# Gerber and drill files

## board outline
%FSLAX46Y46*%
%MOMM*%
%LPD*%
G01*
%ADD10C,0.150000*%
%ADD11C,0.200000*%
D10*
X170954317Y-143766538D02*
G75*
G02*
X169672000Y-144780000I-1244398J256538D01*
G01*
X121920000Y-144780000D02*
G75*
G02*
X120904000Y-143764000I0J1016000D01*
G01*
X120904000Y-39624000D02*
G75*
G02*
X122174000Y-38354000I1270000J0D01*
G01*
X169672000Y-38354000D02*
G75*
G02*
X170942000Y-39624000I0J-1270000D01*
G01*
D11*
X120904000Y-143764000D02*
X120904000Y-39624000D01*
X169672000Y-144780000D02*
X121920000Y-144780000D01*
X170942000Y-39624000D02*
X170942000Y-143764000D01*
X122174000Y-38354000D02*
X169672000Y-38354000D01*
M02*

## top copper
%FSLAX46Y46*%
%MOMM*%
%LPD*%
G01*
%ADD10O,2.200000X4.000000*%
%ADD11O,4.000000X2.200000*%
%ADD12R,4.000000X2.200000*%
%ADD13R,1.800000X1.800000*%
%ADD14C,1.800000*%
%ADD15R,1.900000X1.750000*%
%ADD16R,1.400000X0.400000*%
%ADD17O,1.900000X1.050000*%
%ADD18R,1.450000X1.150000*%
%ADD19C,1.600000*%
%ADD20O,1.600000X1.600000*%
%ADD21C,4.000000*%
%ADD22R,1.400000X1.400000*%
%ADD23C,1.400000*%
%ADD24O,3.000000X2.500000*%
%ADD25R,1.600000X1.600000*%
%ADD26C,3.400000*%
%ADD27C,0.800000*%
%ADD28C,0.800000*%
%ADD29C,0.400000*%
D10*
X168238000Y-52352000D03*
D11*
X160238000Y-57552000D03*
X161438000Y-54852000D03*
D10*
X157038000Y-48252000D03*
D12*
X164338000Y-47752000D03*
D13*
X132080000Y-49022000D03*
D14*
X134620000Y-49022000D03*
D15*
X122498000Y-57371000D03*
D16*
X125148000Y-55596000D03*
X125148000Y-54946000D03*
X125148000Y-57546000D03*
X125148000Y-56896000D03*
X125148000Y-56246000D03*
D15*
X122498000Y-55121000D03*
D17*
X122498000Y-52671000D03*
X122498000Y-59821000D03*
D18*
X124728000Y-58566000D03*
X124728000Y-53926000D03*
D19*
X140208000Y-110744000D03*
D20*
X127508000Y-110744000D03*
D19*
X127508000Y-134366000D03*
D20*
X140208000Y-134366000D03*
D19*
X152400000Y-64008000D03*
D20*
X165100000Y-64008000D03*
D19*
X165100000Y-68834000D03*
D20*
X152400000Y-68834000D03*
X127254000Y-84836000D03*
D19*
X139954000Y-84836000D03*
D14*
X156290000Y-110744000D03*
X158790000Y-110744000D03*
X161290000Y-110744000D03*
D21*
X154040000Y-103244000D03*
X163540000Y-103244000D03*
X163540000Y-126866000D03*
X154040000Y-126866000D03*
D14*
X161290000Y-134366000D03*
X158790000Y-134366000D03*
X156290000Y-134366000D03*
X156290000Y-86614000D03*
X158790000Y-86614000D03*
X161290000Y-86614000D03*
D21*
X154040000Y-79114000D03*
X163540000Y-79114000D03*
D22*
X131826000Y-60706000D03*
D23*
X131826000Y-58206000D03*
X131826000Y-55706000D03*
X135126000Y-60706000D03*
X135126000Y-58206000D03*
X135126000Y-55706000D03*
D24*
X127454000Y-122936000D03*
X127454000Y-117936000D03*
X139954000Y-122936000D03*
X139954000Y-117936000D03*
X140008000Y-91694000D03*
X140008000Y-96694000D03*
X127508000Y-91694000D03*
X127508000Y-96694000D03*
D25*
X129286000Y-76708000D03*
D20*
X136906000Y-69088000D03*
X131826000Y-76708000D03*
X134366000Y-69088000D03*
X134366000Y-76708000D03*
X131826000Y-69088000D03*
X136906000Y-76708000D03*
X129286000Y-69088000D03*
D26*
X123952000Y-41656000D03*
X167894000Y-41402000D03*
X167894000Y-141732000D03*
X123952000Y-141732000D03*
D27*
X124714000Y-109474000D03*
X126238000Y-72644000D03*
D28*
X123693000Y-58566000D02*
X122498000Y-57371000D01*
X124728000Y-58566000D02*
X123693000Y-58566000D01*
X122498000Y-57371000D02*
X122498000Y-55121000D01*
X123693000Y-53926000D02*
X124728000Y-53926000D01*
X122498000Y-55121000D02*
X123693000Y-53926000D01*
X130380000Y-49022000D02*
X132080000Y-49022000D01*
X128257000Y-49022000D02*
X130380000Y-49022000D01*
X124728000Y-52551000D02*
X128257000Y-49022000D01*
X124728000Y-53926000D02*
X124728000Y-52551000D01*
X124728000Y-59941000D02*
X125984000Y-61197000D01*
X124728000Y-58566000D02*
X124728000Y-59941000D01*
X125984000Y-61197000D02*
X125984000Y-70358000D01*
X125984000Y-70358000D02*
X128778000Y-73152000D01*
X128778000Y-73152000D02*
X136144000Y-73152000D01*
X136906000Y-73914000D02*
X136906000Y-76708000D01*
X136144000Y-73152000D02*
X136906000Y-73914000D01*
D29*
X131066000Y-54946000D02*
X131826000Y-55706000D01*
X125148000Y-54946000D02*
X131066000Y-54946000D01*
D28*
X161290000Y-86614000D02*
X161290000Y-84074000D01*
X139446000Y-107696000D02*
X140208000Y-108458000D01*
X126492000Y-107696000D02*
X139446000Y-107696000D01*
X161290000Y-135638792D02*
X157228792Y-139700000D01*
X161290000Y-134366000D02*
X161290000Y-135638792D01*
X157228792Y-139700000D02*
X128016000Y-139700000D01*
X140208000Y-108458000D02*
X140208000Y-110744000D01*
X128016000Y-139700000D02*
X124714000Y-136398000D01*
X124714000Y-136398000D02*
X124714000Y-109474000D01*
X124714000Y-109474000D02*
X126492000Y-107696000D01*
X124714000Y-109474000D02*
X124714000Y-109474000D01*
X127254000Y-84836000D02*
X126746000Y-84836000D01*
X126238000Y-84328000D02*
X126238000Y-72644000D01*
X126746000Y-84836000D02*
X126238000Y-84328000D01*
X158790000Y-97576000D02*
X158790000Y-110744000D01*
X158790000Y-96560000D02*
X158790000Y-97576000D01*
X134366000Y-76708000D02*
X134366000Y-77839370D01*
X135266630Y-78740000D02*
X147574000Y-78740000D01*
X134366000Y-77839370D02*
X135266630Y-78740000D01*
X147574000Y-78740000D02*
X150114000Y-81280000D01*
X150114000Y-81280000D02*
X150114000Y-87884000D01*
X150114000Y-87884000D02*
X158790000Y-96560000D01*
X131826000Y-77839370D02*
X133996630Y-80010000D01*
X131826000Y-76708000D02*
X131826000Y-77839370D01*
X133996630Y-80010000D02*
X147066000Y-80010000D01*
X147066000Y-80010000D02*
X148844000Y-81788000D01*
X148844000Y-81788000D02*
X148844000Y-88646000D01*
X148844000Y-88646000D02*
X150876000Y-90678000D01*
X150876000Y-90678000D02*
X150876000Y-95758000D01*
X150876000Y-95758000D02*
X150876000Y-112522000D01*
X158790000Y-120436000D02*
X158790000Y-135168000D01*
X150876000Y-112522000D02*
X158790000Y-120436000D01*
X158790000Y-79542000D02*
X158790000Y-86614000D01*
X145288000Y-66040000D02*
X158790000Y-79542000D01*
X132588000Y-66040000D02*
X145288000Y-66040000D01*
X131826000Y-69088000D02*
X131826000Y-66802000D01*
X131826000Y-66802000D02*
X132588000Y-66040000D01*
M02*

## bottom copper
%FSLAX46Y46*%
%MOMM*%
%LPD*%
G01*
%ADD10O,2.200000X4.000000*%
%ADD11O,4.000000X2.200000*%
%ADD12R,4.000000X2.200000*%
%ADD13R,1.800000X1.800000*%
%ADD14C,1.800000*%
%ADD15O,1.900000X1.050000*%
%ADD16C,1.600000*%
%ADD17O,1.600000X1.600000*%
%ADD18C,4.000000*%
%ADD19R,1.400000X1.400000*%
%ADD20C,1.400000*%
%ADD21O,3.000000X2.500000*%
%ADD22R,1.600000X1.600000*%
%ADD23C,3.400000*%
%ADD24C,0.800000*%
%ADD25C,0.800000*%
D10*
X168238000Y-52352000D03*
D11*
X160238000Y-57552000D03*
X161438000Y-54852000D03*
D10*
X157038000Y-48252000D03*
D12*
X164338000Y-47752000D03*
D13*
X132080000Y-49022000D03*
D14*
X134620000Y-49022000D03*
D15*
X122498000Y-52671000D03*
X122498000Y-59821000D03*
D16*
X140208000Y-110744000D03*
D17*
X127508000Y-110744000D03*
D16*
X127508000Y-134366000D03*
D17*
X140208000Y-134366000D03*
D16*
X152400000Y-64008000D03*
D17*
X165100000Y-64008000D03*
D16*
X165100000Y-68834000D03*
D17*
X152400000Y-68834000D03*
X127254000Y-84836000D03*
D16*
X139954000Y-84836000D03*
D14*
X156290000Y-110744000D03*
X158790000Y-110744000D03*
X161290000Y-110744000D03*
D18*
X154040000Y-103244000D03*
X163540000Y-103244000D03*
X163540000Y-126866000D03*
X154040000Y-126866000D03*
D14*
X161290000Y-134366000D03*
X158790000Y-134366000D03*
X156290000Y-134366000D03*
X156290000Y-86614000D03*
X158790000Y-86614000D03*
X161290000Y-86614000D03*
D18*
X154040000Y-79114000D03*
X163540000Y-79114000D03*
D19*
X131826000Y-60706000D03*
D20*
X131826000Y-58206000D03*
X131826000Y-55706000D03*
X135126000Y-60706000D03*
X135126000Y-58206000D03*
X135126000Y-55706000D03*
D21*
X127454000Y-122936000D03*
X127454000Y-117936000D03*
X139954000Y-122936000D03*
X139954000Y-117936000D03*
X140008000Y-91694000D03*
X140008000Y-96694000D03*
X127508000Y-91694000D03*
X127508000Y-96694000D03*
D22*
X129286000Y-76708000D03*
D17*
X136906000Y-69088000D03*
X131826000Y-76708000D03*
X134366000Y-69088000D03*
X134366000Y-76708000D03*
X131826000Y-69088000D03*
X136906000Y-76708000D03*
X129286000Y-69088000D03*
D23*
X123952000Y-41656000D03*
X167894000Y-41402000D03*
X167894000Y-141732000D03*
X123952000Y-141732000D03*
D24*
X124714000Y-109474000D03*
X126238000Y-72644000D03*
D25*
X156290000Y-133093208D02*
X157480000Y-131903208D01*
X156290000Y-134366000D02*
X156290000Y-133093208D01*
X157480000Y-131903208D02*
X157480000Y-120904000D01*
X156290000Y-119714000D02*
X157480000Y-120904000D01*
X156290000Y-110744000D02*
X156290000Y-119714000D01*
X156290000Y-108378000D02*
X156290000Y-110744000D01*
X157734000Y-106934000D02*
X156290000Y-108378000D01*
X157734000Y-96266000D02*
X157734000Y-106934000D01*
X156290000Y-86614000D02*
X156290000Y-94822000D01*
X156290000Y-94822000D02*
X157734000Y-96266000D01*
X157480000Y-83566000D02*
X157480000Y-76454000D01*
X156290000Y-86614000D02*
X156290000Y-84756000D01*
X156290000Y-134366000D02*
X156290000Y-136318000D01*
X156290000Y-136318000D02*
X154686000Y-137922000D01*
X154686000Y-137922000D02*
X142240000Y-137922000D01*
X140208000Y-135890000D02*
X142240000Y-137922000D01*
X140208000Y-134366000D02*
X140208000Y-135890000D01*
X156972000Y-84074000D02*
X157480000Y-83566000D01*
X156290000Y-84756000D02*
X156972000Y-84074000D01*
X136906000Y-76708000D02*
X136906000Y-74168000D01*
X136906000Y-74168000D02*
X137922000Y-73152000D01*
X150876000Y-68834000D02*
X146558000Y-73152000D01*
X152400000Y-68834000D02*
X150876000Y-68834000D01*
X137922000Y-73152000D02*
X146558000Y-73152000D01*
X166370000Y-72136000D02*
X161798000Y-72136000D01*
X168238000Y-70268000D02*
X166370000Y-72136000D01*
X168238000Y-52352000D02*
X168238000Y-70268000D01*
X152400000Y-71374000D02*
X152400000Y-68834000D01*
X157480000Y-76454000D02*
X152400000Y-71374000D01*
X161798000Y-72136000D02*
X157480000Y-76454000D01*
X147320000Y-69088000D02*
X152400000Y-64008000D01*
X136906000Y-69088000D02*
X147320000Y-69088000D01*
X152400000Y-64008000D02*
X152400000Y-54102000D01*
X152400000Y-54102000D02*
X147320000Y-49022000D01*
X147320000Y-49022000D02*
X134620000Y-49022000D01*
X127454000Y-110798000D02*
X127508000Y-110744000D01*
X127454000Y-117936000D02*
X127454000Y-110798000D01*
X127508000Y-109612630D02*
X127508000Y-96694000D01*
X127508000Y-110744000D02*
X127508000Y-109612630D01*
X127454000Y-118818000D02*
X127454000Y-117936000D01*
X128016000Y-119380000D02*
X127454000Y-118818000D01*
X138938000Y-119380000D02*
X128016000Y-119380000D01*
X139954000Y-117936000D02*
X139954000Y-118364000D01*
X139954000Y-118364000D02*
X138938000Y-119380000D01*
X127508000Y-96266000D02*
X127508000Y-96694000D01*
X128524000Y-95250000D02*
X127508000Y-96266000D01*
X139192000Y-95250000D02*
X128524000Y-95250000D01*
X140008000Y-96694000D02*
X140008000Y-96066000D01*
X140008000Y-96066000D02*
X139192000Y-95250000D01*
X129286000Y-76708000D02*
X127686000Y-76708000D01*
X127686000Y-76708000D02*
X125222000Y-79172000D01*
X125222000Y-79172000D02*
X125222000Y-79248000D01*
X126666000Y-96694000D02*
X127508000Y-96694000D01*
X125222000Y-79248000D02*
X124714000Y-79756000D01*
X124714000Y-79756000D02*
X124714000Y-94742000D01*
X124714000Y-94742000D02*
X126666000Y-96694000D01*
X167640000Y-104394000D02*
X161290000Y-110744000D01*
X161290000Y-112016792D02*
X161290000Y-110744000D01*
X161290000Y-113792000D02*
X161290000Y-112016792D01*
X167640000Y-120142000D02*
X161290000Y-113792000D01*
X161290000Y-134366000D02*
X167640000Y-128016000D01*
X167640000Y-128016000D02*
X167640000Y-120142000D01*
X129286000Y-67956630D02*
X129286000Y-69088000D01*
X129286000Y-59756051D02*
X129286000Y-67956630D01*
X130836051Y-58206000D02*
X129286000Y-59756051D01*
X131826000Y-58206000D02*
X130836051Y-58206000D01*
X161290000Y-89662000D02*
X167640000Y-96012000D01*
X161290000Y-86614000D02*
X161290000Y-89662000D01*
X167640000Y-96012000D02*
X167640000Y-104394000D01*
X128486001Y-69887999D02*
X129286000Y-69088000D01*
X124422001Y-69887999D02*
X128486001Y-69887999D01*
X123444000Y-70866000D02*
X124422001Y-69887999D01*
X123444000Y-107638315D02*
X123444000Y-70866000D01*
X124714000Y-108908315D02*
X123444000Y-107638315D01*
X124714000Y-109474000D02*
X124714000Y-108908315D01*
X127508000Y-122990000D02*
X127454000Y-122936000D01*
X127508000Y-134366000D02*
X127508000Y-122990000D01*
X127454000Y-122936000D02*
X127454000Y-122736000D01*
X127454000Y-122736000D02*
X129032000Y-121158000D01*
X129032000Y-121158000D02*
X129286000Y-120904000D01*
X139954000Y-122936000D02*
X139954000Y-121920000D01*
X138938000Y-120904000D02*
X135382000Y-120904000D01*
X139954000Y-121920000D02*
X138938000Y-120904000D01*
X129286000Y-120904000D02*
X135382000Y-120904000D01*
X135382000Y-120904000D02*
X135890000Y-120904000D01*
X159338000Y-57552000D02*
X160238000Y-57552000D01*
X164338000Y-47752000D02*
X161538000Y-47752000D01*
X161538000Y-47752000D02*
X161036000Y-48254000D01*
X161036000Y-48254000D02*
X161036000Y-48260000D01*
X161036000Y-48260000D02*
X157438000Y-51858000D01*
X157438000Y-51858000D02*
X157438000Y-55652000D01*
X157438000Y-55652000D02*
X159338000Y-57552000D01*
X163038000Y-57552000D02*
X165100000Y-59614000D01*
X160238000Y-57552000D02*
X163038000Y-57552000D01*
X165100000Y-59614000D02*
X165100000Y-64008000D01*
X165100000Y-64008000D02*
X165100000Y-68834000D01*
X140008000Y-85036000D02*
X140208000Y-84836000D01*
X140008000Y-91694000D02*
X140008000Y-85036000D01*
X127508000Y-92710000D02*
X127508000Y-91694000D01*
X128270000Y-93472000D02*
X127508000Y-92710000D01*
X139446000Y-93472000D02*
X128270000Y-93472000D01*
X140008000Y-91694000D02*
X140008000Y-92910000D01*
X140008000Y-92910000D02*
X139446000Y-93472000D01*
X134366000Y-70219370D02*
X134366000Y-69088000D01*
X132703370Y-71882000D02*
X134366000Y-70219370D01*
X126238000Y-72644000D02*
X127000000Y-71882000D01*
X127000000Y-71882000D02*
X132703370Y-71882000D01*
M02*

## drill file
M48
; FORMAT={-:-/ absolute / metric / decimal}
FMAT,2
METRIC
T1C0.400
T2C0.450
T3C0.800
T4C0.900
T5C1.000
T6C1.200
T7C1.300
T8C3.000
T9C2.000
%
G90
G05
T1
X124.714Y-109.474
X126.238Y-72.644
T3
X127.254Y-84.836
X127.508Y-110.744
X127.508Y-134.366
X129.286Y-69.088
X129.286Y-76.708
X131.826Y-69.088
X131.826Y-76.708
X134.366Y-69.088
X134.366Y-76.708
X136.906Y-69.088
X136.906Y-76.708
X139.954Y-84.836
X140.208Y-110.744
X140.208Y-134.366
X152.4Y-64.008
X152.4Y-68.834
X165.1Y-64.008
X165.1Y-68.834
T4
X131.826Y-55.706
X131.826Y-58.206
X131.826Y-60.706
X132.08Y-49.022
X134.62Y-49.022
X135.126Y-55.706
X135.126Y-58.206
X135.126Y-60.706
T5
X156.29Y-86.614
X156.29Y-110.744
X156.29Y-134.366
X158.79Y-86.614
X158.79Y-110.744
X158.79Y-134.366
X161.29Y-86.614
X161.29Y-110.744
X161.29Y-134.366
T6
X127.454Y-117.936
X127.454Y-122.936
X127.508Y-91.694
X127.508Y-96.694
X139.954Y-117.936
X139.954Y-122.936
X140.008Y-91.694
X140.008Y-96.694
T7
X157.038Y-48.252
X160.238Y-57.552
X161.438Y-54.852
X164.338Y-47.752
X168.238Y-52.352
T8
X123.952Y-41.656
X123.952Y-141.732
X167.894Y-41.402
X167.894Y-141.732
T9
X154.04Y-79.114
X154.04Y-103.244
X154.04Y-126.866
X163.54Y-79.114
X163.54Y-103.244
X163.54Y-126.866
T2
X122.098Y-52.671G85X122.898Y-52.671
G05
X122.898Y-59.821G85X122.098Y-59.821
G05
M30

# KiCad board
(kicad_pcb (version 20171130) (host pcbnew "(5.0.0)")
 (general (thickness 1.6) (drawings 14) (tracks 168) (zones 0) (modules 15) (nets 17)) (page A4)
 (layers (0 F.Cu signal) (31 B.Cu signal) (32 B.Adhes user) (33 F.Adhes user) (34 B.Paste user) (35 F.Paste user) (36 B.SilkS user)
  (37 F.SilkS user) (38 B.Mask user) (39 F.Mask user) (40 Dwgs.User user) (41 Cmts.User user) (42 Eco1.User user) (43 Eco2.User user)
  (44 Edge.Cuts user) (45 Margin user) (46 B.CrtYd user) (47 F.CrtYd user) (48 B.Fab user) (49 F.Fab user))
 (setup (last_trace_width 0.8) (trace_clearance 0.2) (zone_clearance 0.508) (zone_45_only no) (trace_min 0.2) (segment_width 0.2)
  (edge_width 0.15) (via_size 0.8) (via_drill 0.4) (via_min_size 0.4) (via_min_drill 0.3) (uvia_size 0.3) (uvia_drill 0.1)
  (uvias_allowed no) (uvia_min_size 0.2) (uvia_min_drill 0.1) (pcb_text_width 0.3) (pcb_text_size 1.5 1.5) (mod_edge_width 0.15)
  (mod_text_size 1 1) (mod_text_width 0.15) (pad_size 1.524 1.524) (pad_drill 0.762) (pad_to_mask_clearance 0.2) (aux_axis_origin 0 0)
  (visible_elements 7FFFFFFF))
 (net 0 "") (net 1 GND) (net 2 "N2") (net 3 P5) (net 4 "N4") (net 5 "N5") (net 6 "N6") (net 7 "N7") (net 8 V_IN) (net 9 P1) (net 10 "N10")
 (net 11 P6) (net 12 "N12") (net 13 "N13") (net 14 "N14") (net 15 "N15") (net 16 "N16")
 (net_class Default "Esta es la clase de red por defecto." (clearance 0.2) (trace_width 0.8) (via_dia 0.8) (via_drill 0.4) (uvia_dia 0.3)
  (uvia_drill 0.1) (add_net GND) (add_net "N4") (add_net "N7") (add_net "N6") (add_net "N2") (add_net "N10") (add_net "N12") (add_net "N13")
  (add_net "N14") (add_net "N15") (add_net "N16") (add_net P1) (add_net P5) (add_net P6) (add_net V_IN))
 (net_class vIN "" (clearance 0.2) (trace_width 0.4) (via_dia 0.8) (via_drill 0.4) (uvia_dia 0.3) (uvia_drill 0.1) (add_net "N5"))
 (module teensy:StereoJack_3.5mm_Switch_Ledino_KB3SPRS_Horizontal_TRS (layer F.Cu) (at 164.338 47.752 180)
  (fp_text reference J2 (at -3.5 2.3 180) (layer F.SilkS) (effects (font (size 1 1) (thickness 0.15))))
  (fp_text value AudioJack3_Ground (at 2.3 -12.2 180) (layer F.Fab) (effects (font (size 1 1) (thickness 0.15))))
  (pad S thru_hole oval (at -3.9 -4.6 180) (size 2.2 4) (drill 1.3) (layers *.Cu *.Mask) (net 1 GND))
  (pad T thru_hole oval (at 4.1 -9.8 180) (size 4 2.2) (drill 1.3) (layers *.Cu *.Mask) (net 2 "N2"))
  (pad 5 thru_hole oval (at 2.9 -7.1 180) (size 4 2.2) (drill 1.3) (layers *.Cu *.Mask))
  (pad 4 thru_hole oval (at 7.3 -0.5 270) (size 4 2.2) (drill 1.3) (layers *.Cu *.Mask))
  (pad R thru_hole rect (at 0 0 180) (size 4 2.2) (drill 1.3) (layers *.Cu *.Mask) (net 2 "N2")))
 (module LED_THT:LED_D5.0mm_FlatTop (layer F.Cu) (at 132.08 49.022)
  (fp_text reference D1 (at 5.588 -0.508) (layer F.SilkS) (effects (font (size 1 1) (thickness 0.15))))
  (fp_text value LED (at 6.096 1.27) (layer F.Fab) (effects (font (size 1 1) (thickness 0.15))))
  (pad 1 thru_hole rect (at 0 0) (size 1.8 1.8) (drill 0.9) (layers *.Cu *.Mask) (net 1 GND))
  (pad 2 thru_hole circle (at 2.54 0) (size 1.8 1.8) (drill 0.9) (layers *.Cu *.Mask) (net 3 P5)))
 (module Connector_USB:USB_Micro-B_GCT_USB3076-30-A (layer F.Cu) (at 123.698 56.246 270)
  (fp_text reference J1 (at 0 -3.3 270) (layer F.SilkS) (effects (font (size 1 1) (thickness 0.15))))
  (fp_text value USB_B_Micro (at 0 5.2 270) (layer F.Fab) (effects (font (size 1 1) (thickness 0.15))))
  (pad 6 smd rect (at 1.125 1.2 270) (size 1.75 1.9) (layers F.Cu F.Paste F.Mask) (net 1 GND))
  (pad 2 smd rect (at -0.65 -1.45 270) (size 0.4 1.4) (layers F.Cu F.Paste F.Mask) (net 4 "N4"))
  (pad 1 smd rect (at -1.3 -1.45 270) (size 0.4 1.4) (layers F.Cu F.Paste F.Mask) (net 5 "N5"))
  (pad 5 smd rect (at 1.3 -1.45 270) (size 0.4 1.4) (layers F.Cu F.Paste F.Mask) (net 1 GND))
  (pad 4 smd rect (at 0.65 -1.45 270) (size 0.4 1.4) (layers F.Cu F.Paste F.Mask) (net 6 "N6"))
  (pad 3 smd rect (at 0 -1.45 270) (size 0.4 1.4) (layers F.Cu F.Paste F.Mask) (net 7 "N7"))
  (pad 6 smd rect (at -1.125 1.2 270) (size 1.75 1.9) (layers F.Cu F.Paste F.Mask) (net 1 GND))
  (pad 6 thru_hole oval (at -3.575 1.2 90) (size 1.05 1.9) (drill oval 0.45 1.25) (layers *.Cu *.Mask) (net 1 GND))
  (pad 6 thru_hole oval (at 3.575 1.2 270) (size 1.05 1.9) (drill oval 0.45 1.25) (layers *.Cu *.Mask) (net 1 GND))
  (pad 6 smd rect (at 2.32 -1.03 270) (size 1.15 1.45) (layers F.Cu F.Paste F.Mask) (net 1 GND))
  (pad 6 smd rect (at -2.32 -1.03 270) (size 1.15 1.45) (layers F.Cu F.Paste F.Mask) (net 1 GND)))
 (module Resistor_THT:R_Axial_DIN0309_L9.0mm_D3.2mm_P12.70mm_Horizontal (layer F.Cu) (at 140.208 110.744 180)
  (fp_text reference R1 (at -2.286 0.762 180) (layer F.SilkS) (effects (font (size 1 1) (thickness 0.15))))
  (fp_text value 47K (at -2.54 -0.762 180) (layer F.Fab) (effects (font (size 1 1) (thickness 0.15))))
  (pad 1 thru_hole circle (at 0 0 180) (size 1.6 1.6) (drill 0.8) (layers *.Cu *.Mask) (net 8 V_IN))
  (pad 2 thru_hole oval (at 12.7 0 180) (size 1.6 1.6) (drill 0.8) (layers *.Cu *.Mask) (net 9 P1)))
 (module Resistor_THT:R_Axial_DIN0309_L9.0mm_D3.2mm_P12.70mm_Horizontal (layer F.Cu) (at 127.508 134.366)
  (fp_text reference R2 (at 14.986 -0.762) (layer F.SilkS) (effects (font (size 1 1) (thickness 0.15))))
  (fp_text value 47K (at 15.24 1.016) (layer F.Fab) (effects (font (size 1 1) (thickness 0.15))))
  (pad 1 thru_hole circle (at 0 0) (size 1.6 1.6) (drill 0.8) (layers *.Cu *.Mask) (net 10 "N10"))
  (pad 2 thru_hole oval (at 12.7 0) (size 1.6 1.6) (drill 0.8) (layers *.Cu *.Mask) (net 1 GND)))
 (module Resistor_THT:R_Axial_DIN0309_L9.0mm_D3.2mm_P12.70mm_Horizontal (layer F.Cu) (at 152.4 64.008)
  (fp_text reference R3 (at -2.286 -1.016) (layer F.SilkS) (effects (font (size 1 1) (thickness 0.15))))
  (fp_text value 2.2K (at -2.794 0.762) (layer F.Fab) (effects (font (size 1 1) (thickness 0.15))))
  (pad 1 thru_hole circle (at 0 0) (size 1.6 1.6) (drill 0.8) (layers *.Cu *.Mask) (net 3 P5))
  (pad 2 thru_hole oval (at 12.7 0) (size 1.6 1.6) (drill 0.8) (layers *.Cu *.Mask) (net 2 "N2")))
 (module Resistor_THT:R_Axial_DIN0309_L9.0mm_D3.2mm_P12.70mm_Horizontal (layer F.Cu) (at 165.1 68.834 180)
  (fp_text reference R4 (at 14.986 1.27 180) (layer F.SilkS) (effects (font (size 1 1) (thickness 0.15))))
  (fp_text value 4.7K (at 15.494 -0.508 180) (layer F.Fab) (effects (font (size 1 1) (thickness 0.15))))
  (pad 1 thru_hole circle (at 0 0 180) (size 1.6 1.6) (drill 0.8) (layers *.Cu *.Mask) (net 2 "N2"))
  (pad 2 thru_hole oval (at 12.7 0 180) (size 1.6 1.6) (drill 0.8) (layers *.Cu *.Mask) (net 1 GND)))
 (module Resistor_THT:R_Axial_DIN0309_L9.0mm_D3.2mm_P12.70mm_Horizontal (layer F.Cu) (at 139.954 84.836 180)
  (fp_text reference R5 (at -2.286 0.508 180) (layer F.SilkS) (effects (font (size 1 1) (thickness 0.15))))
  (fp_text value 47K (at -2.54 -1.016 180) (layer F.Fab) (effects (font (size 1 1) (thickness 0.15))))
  (pad 2 thru_hole oval (at 12.7 0 180) (size 1.6 1.6) (drill 0.8) (layers *.Cu *.Mask) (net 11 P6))
  (pad 1 thru_hole circle (at 0 0 180) (size 1.6 1.6) (drill 0.8) (layers *.Cu *.Mask) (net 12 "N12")))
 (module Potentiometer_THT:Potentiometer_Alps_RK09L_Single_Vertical (layer F.Cu) (at 161.29 110.744 90)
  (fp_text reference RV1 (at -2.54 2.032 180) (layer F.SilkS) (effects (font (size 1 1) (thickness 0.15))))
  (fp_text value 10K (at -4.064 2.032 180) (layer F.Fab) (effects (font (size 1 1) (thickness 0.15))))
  (pad 3 thru_hole circle (at 0 -5 90) (size 1.8 1.8) (drill 1) (layers *.Cu *.Mask) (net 1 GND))
  (pad 2 thru_hole circle (at 0 -2.5 90) (size 1.8 1.8) (drill 1) (layers *.Cu *.Mask) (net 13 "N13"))
  (pad 1 thru_hole circle (at 0 0 90) (size 1.8 1.8) (drill 1) (layers *.Cu *.Mask) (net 8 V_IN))
  (pad "" np_thru_hole circle (at 7.5 -7.25 90) (size 4 4) (drill 2) (layers *.Cu *.Mask))
  (pad "" np_thru_hole circle (at 7.5 2.25 90) (size 4 4) (drill 2) (layers *.Cu *.Mask)))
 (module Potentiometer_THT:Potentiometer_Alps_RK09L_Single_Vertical (layer F.Cu) (at 161.29 134.366 90)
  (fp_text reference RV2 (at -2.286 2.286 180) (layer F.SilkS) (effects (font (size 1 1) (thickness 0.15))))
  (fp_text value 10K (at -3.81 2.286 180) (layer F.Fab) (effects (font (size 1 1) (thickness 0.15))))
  (pad "" np_thru_hole circle (at 7.5 2.25 90) (size 4 4) (drill 2) (layers *.Cu *.Mask))
  (pad "" np_thru_hole circle (at 7.5 -7.25 90) (size 4 4) (drill 2) (layers *.Cu *.Mask))
  (pad 1 thru_hole circle (at 0 0 90) (size 1.8 1.8) (drill 1) (layers *.Cu *.Mask) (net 8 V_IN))
  (pad 2 thru_hole circle (at 0 -2.5 90) (size 1.8 1.8) (drill 1) (layers *.Cu *.Mask) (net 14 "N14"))
  (pad 3 thru_hole circle (at 0 -5 90) (size 1.8 1.8) (drill 1) (layers *.Cu *.Mask) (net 1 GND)))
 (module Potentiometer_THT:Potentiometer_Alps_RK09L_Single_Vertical (layer F.Cu) (at 161.29 86.614 90)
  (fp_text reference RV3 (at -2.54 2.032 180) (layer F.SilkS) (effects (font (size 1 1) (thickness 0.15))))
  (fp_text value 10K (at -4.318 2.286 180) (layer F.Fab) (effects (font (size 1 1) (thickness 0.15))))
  (pad 3 thru_hole circle (at 0 -5 90) (size 1.8 1.8) (drill 1) (layers *.Cu *.Mask) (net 1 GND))
  (pad 2 thru_hole circle (at 0 -2.5 90) (size 1.8 1.8) (drill 1) (layers *.Cu *.Mask) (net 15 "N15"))
  (pad 1 thru_hole circle (at 0 0 90) (size 1.8 1.8) (drill 1) (layers *.Cu *.Mask) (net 8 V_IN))
  (pad "" np_thru_hole circle (at 7.5 -7.25 90) (size 4 4) (drill 2) (layers *.Cu *.Mask))
  (pad "" np_thru_hole circle (at 7.5 2.25 90) (size 4 4) (drill 2) (layers *.Cu *.Mask)))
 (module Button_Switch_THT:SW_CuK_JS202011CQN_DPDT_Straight (layer F.Cu) (at 131.826 60.706 90)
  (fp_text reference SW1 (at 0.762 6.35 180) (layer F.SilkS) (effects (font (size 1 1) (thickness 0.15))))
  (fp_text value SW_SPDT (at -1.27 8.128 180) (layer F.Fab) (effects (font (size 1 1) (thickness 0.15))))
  (pad 1 thru_hole rect (at 0 0 90) (size 1.4 1.4) (drill 0.9) (layers *.Cu *.Mask) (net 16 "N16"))
  (pad 2 thru_hole circle (at 2.5 0 90) (size 1.4 1.4) (drill 0.9) (layers *.Cu *.Mask) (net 8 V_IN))
  (pad 3 thru_hole circle (at 5 0 90) (size 1.4 1.4) (drill 0.9) (layers *.Cu *.Mask) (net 5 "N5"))
  (pad 4 thru_hole circle (at 0 3.3 90) (size 1.4 1.4) (drill 0.9) (layers *.Cu *.Mask))
  (pad 5 thru_hole circle (at 2.5 3.3 90) (size 1.4 1.4) (drill 0.9) (layers *.Cu *.Mask))
  (pad 6 thru_hole circle (at 5 3.3 90) (size 1.4 1.4) (drill 0.9) (layers *.Cu *.Mask)))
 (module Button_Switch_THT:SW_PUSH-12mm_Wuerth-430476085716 (layer F.Cu) (at 139.954 122.936 180)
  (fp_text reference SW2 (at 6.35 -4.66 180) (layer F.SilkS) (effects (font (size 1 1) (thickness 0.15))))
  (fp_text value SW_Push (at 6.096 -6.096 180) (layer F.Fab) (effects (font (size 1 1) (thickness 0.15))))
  (pad 1 thru_hole oval (at 12.5 0 180) (size 3 2.5) (drill 1.2) (layers *.Cu *.Mask) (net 10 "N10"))
  (pad 2 thru_hole oval (at 12.5 5 180) (size 3 2.5) (drill 1.2) (layers *.Cu *.Mask) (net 9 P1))
  (pad 1 thru_hole oval (at 0 0 180) (size 3 2.5) (drill 1.2) (layers *.Cu *.Mask) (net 10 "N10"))
  (pad 2 thru_hole oval (at 0 5 180) (size 3 2.5) (drill 1.2) (layers *.Cu *.Mask) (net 9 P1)))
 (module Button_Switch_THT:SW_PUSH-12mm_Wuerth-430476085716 (layer F.Cu) (at 127.508 91.694)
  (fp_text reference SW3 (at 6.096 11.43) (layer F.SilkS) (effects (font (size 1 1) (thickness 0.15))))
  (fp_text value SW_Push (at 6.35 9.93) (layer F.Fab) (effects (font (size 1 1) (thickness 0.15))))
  (pad 1 thru_hole oval (at 12.5 0) (size 3 2.5) (drill 1.2) (layers *.Cu *.Mask) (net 12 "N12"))
  (pad 2 thru_hole oval (at 12.5 5) (size 3 2.5) (drill 1.2) (layers *.Cu *.Mask) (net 9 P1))
  (pad 1 thru_hole oval (at 0 0) (size 3 2.5) (drill 1.2) (layers *.Cu *.Mask) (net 12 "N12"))
  (pad 2 thru_hole oval (at 0 5) (size 3 2.5) (drill 1.2) (layers *.Cu *.Mask) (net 9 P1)))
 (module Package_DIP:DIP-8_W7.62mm (layer F.Cu) (at 129.286 76.708 90)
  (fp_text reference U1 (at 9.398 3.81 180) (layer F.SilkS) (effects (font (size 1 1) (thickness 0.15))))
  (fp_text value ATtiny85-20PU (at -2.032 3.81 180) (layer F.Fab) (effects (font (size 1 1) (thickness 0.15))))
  (pad 1 thru_hole rect (at 0 0 90) (size 1.6 1.6) (drill 0.8) (layers *.Cu *.Mask) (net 9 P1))
  (pad 5 thru_hole oval (at 7.62 7.62 90) (size 1.6 1.6) (drill 0.8) (layers *.Cu *.Mask) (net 3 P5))
  (pad 2 thru_hole oval (at 0 2.54 90) (size 1.6 1.6) (drill 0.8) (layers *.Cu *.Mask) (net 14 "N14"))
  (pad 6 thru_hole oval (at 7.62 5.08 90) (size 1.6 1.6) (drill 0.8) (layers *.Cu *.Mask) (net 11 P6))
  (pad 3 thru_hole oval (at 0 5.08 90) (size 1.6 1.6) (drill 0.8) (layers *.Cu *.Mask) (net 13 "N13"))
  (pad 7 thru_hole oval (at 7.62 2.54 90) (size 1.6 1.6) (drill 0.8) (layers *.Cu *.Mask) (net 15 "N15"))
  (pad 4 thru_hole oval (at 0 7.62 90) (size 1.6 1.6) (drill 0.8) (layers *.Cu *.Mask) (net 1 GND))
  (pad 8 thru_hole oval (at 7.62 0 90) (size 1.6 1.6) (drill 0.8) (layers *.Cu *.Mask) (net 8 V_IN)))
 (gr_arc (start 169.709919 143.51) (end 169.672 144.78) (angle -80.06160025) (layer Edge.Cuts) (width 0.15))
 (gr_arc (start 121.92 143.764) (end 120.904 143.764) (angle -90) (layer Edge.Cuts) (width 0.15))
 (gr_arc (start 122.174 39.624) (end 122.174 38.354) (angle -90) (layer Edge.Cuts) (width 0.15))
 (gr_arc (start 169.672 39.624) (end 170.942 39.624) (angle -90) (layer Edge.Cuts) (width 0.15))
 (gr_line (start 120.904 143.764) (end 120.904 39.624) (layer Edge.Cuts) (width 0.2))
 (gr_line (start 169.672 144.78) (end 121.92 144.78) (layer Edge.Cuts) (width 0.2))
 (gr_line (start 170.942 39.624) (end 170.942 143.764) (layer Edge.Cuts) (width 0.2))
 (gr_line (start 122.174 38.354) (end 169.672 38.354) (layer Edge.Cuts) (width 0.2))
 (via (at 123.952 41.656) (size 3.4) (drill 3) (layers F.Cu B.Cu) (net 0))
 (via (at 167.894 41.402) (size 3.4) (drill 3) (layers F.Cu B.Cu) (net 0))
 (via (at 167.894 141.732) (size 3.4) (drill 3) (layers F.Cu B.Cu) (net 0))
 (via (at 123.952 141.732) (size 3.4) (drill 3) (layers F.Cu B.Cu) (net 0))
 (segment (start 123.693 58.566) (end 122.498 57.371) (width 0.8) (layer F.Cu) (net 1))
 (segment (start 124.728 58.566) (end 123.693 58.566) (width 0.8) (layer F.Cu) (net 1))
 (segment (start 122.498 57.371) (end 122.498 55.121) (width 0.8) (layer F.Cu) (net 1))
 (segment (start 123.693 53.926) (end 124.728 53.926) (width 0.8) (layer F.Cu) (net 1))
 (segment (start 122.498 55.121) (end 123.693 53.926) (width 0.8) (layer F.Cu) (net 1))
 (segment (start 130.38 49.022) (end 132.08 49.022) (width 0.8) (layer F.Cu) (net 1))
 (segment (start 128.257 49.022) (end 130.38 49.022) (width 0.8) (layer F.Cu) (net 1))
 (segment (start 124.728 52.551) (end 128.257 49.022) (width 0.8) (layer F.Cu) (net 1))
 (segment (start 124.728 53.926) (end 124.728 52.551) (width 0.8) (layer F.Cu) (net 1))
 (segment (start 124.728 59.941) (end 125.984 61.197) (width 0.8) (layer F.Cu) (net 1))
 (segment (start 124.728 58.566) (end 124.728 59.941) (width 0.8) (layer F.Cu) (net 1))
 (segment (start 125.984 61.197) (end 125.984 70.358) (width 0.8) (layer F.Cu) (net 1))
 (segment (start 125.984 70.358) (end 128.778 73.152) (width 0.8) (layer F.Cu) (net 1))
 (segment (start 128.778 73.152) (end 136.144 73.152) (width 0.8) (layer F.Cu) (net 1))
 (segment (start 136.906 73.914) (end 136.906 76.708) (width 0.8) (layer F.Cu) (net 1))
 (segment (start 136.144 73.152) (end 136.906 73.914) (width 0.8) (layer F.Cu) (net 1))
 (segment (start 156.29 133.093208) (end 157.48 131.903208) (width 0.8) (layer B.Cu) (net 1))
 (segment (start 156.29 134.366) (end 156.29 133.093208) (width 0.8) (layer B.Cu) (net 1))
 (segment (start 157.48 131.903208) (end 157.48 120.904) (width 0.8) (layer B.Cu) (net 1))
 (segment (start 156.29 119.714) (end 157.48 120.904) (width 0.8) (layer B.Cu) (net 1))
 (segment (start 156.29 110.744) (end 156.29 119.714) (width 0.8) (layer B.Cu) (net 1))
 (segment (start 156.29 108.378) (end 156.29 110.744) (width 0.8) (layer B.Cu) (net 1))
 (segment (start 157.734 106.934) (end 156.29 108.378) (width 0.8) (layer B.Cu) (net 1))
 (segment (start 157.734 96.266) (end 157.734 106.934) (width 0.8) (layer B.Cu) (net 1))
 (segment (start 156.29 86.614) (end 156.29 94.822) (width 0.8) (layer B.Cu) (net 1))
 (segment (start 156.29 94.822) (end 157.734 96.266) (width 0.8) (layer B.Cu) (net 1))
 (segment (start 157.48 83.566) (end 157.48 76.454) (width 0.8) (layer B.Cu) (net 1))
 (segment (start 156.29 86.614) (end 156.29 84.756) (width 0.8) (layer B.Cu) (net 1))
 (segment (start 156.29 134.366) (end 156.29 136.318) (width 0.8) (layer B.Cu) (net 1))
 (segment (start 156.29 136.318) (end 154.686 137.922) (width 0.8) (layer B.Cu) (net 1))
 (segment (start 154.686 137.922) (end 142.24 137.922) (width 0.8) (layer B.Cu) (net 1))
 (segment (start 140.208 135.89) (end 142.24 137.922) (width 0.8) (layer B.Cu) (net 1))
 (segment (start 140.208 134.366) (end 140.208 135.89) (width 0.8) (layer B.Cu) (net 1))
 (segment (start 156.972 84.074) (end 157.48 83.566) (width 0.8) (layer B.Cu) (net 1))
 (segment (start 156.29 84.756) (end 156.972 84.074) (width 0.8) (layer B.Cu) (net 1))
 (segment (start 136.906 76.708) (end 136.906 74.168) (width 0.8) (layer B.Cu) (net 1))
 (segment (start 136.906 74.168) (end 137.922 73.152) (width 0.8) (layer B.Cu) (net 1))
 (segment (start 150.876 68.834) (end 146.558 73.152) (width 0.8) (layer B.Cu) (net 1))
 (segment (start 152.4 68.834) (end 150.876 68.834) (width 0.8) (layer B.Cu) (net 1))
 (segment (start 137.922 73.152) (end 146.558 73.152) (width 0.8) (layer B.Cu) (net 1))
 (segment (start 166.37 72.136) (end 161.798 72.136) (width 0.8) (layer B.Cu) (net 1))
 (segment (start 168.238 70.268) (end 166.37 72.136) (width 0.8) (layer B.Cu) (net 1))
 (segment (start 168.238 52.352) (end 168.238 70.268) (width 0.8) (layer B.Cu) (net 1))
 (segment (start 152.4 71.374) (end 152.4 68.834) (width 0.8) (layer B.Cu) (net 1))
 (segment (start 157.48 76.454) (end 152.4 71.374) (width 0.8) (layer B.Cu) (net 1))
 (segment (start 161.798 72.136) (end 157.48 76.454) (width 0.8) (layer B.Cu) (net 1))
 (segment (start 147.32 69.088) (end 152.4 64.008) (width 0.8) (layer B.Cu) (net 3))
 (segment (start 136.906 69.088) (end 147.32 69.088) (width 0.8) (layer B.Cu) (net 3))
 (segment (start 152.4 64.008) (end 152.4 54.102) (width 0.8) (layer B.Cu) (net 3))
 (segment (start 152.4 54.102) (end 147.32 49.022) (width 0.8) (layer B.Cu) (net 3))
 (segment (start 147.32 49.022) (end 134.62 49.022) (width 0.8) (layer B.Cu) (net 3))
 (segment (start 131.066 54.946) (end 131.826 55.706) (width 0.4) (layer F.Cu) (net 5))
 (segment (start 125.148 54.946) (end 131.066 54.946) (width 0.4) (layer F.Cu) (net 5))
 (segment (start 127.454 110.798) (end 127.508 110.744) (width 0.8) (layer B.Cu) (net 9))
 (segment (start 127.454 117.936) (end 127.454 110.798) (width 0.8) (layer B.Cu) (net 9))
 (segment (start 127.508 109.61263) (end 127.508 96.694) (width 0.8) (layer B.Cu) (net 9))
 (segment (start 127.508 110.744) (end 127.508 109.61263) (width 0.8) (layer B.Cu) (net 9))
 (segment (start 127.454 118.818) (end 127.454 117.936) (width 0.8) (layer B.Cu) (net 9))
 (segment (start 128.016 119.38) (end 127.454 118.818) (width 0.8) (layer B.Cu) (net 9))
 (segment (start 138.938 119.38) (end 128.016 119.38) (width 0.8) (layer B.Cu) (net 9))
 (segment (start 139.954 117.936) (end 139.954 118.364) (width 0.8) (layer B.Cu) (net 9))
 (segment (start 139.954 118.364) (end 138.938 119.38) (width 0.8) (layer B.Cu) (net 9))
 (segment (start 127.508 96.266) (end 127.508 96.694) (width 0.8) (layer B.Cu) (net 9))
 (segment (start 128.524 95.25) (end 127.508 96.266) (width 0.8) (layer B.Cu) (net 9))
 (segment (start 139.192 95.25) (end 128.524 95.25) (width 0.8) (layer B.Cu) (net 9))
 (segment (start 140.008 96.694) (end 140.008 96.066) (width 0.8) (layer B.Cu) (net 9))
 (segment (start 140.008 96.066) (end 139.192 95.25) (width 0.8) (layer B.Cu) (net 9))
 (segment (start 129.286 76.708) (end 127.686 76.708) (width 0.8) (layer B.Cu) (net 9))
 (segment (start 127.686 76.708) (end 125.222 79.172) (width 0.8) (layer B.Cu) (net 9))
 (segment (start 125.222 79.172) (end 125.222 79.248) (width 0.8) (layer B.Cu) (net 9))
 (segment (start 126.666 96.694) (end 127.508 96.694) (width 0.8) (layer B.Cu) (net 9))
 (segment (start 125.222 79.248) (end 124.714 79.756) (width 0.8) (layer B.Cu) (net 9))
 (segment (start 124.714 79.756) (end 124.714 94.742) (width 0.8) (layer B.Cu) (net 9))
 (segment (start 124.714 94.742) (end 126.666 96.694) (width 0.8) (layer B.Cu) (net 9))
 (segment (start 167.64 104.394) (end 161.29 110.744) (width 0.8) (layer B.Cu) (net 8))
 (segment (start 161.29 112.016792) (end 161.29 110.744) (width 0.8) (layer B.Cu) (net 8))
 (segment (start 161.29 113.792) (end 161.29 112.016792) (width 0.8) (layer B.Cu) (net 8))
 (segment (start 167.64 120.142) (end 161.29 113.792) (width 0.8) (layer B.Cu) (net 8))
 (segment (start 161.29 134.366) (end 167.64 128.016) (width 0.8) (layer B.Cu) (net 8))
 (segment (start 167.64 128.016) (end 167.64 120.142) (width 0.8) (layer B.Cu) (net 8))
 (segment (start 129.286 67.95663) (end 129.286 69.088) (width 0.8) (layer B.Cu) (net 8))
 (segment (start 129.286 59.756051) (end 129.286 67.95663) (width 0.8) (layer B.Cu) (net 8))
 (segment (start 130.836051 58.206) (end 129.286 59.756051) (width 0.8) (layer B.Cu) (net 8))
 (segment (start 131.826 58.206) (end 130.836051 58.206) (width 0.8) (layer B.Cu) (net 8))
 (segment (start 161.29 86.614) (end 161.29 84.074) (width 0.8) (layer F.Cu) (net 8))
 (segment (start 161.29 89.662) (end 167.64 96.012) (width 0.8) (layer B.Cu) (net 8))
 (segment (start 161.29 86.614) (end 161.29 89.662) (width 0.8) (layer B.Cu) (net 8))
 (segment (start 167.64 96.012) (end 167.64 104.394) (width 0.8) (layer B.Cu) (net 8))
 (segment (start 139.446 107.696) (end 140.208 108.458) (width 0.8) (layer F.Cu) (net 8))
 (segment (start 126.492 107.696) (end 139.446 107.696) (width 0.8) (layer F.Cu) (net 8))
 (segment (start 161.29 135.638792) (end 157.228792 139.7) (width 0.8) (layer F.Cu) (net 8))
 (segment (start 161.29 134.366) (end 161.29 135.638792) (width 0.8) (layer F.Cu) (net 8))
 (segment (start 157.228792 139.7) (end 128.016 139.7) (width 0.8) (layer F.Cu) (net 8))
 (segment (start 140.208 108.458) (end 140.208 110.744) (width 0.8) (layer F.Cu) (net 8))
 (segment (start 128.016 139.7) (end 124.714 136.398) (width 0.8) (layer F.Cu) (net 8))
 (segment (start 124.714 136.398) (end 124.714 109.474) (width 0.8) (layer F.Cu) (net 8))
 (segment (start 124.714 109.474) (end 126.492 107.696) (width 0.8) (layer F.Cu) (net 8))
 (segment (start 124.714 109.474) (end 124.714 109.474) (width 0.8) (layer F.Cu) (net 8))
 (via (at 124.714 109.474) (size 0.8) (drill 0.4) (layers F.Cu B.Cu) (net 8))
 (segment (start 128.486001 69.887999) (end 129.286 69.088) (width 0.8) (layer B.Cu) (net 8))
 (segment (start 124.422001 69.887999) (end 128.486001 69.887999) (width 0.8) (layer B.Cu) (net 8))
 (segment (start 123.444 70.866) (end 124.422001 69.887999) (width 0.8) (layer B.Cu) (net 8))
 (segment (start 123.444 107.638315) (end 123.444 70.866) (width 0.8) (layer B.Cu) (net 8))
 (segment (start 124.714 108.908315) (end 123.444 107.638315) (width 0.8) (layer B.Cu) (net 8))
 (segment (start 124.714 109.474) (end 124.714 108.908315) (width 0.8) (layer B.Cu) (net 8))
 (segment (start 127.508 122.99) (end 127.454 122.936) (width 0.8) (layer B.Cu) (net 10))
 (segment (start 127.508 134.366) (end 127.508 122.99) (width 0.8) (layer B.Cu) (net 10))
 (segment (start 127.454 122.936) (end 127.454 122.736) (width 0.8) (layer B.Cu) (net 10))
 (segment (start 127.454 122.736) (end 129.032 121.158) (width 0.8) (layer B.Cu) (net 10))
 (segment (start 129.032 121.158) (end 129.286 120.904) (width 0.8) (layer B.Cu) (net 10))
 (segment (start 139.954 122.936) (end 139.954 121.92) (width 0.8) (layer B.Cu) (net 10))
 (segment (start 138.938 120.904) (end 135.382 120.904) (width 0.8) (layer B.Cu) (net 10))
 (segment (start 139.954 121.92) (end 138.938 120.904) (width 0.8) (layer B.Cu) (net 10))
 (segment (start 129.286 120.904) (end 135.382 120.904) (width 0.8) (layer B.Cu) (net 10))
 (segment (start 135.382 120.904) (end 135.89 120.904) (width 0.8) (layer B.Cu) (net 10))
 (segment (start 159.338 57.552) (end 160.238 57.552) (width 0.8) (layer B.Cu) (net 2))
 (segment (start 164.338 47.752) (end 161.538 47.752) (width 0.8) (layer B.Cu) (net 2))
 (segment (start 161.538 47.752) (end 161.036 48.254) (width 0.8) (layer B.Cu) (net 2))
 (segment (start 161.036 48.254) (end 161.036 48.26) (width 0.8) (layer B.Cu) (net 2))
 (segment (start 161.036 48.26) (end 157.438 51.858) (width 0.8) (layer B.Cu) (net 2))
 (segment (start 157.438 51.858) (end 157.438 55.652) (width 0.8) (layer B.Cu) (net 2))
 (segment (start 157.438 55.652) (end 159.338 57.552) (width 0.8) (layer B.Cu) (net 2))
 (segment (start 163.038 57.552) (end 165.1 59.614) (width 0.8) (layer B.Cu) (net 2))
 (segment (start 160.238 57.552) (end 163.038 57.552) (width 0.8) (layer B.Cu) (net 2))
 (segment (start 165.1 59.614) (end 165.1 64.008) (width 0.8) (layer B.Cu) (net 2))
 (segment (start 165.1 64.008) (end 165.1 68.834) (width 0.8) (layer B.Cu) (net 2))
 (segment (start 140.008 85.036) (end 140.208 84.836) (width 0.8) (layer B.Cu) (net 12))
 (segment (start 140.008 91.694) (end 140.008 85.036) (width 0.8) (layer B.Cu) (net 12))
 (segment (start 127.508 92.71) (end 127.508 91.694) (width 0.8) (layer B.Cu) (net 12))
 (segment (start 128.27 93.472) (end 127.508 92.71) (width 0.8) (layer B.Cu) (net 12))
 (segment (start 139.446 93.472) (end 128.27 93.472) (width 0.8) (layer B.Cu) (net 12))
 (segment (start 140.008 91.694) (end 140.008 92.91) (width 0.8) (layer B.Cu) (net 12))
 (segment (start 140.008 92.91) (end 139.446 93.472) (width 0.8) (layer B.Cu) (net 12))
 (via (at 126.238 72.644) (size 0.8) (drill 0.4) (layers F.Cu B.Cu) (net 11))
 (segment (start 127.254 84.836) (end 126.746 84.836) (width 0.8) (layer F.Cu) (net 11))
 (segment (start 126.238 84.328) (end 126.238 72.644) (width 0.8) (layer F.Cu) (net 11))
 (segment (start 126.746 84.836) (end 126.238 84.328) (width 0.8) (layer F.Cu) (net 11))
 (segment (start 134.366 70.21937) (end 134.366 69.088) (width 0.8) (layer B.Cu) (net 11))
 (segment (start 132.70337 71.882) (end 134.366 70.21937) (width 0.8) (layer B.Cu) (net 11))
 (segment (start 126.238 72.644) (end 127 71.882) (width 0.8) (layer B.Cu) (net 11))
 (segment (start 127 71.882) (end 132.70337 71.882) (width 0.8) (layer B.Cu) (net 11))
 (segment (start 158.79 97.576) (end 158.79 110.744) (width 0.8) (layer F.Cu) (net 13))
 (segment (start 158.79 96.56) (end 158.79 97.576) (width 0.8) (layer F.Cu) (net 13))
 (segment (start 134.366 76.708) (end 134.366 77.83937) (width 0.8) (layer F.Cu) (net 13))
 (segment (start 135.26663 78.74) (end 147.574 78.74) (width 0.8) (layer F.Cu) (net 13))
 (segment (start 134.366 77.83937) (end 135.26663 78.74) (width 0.8) (layer F.Cu) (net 13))
 (segment (start 147.574 78.74) (end 150.114 81.28) (width 0.8) (layer F.Cu) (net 13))
 (segment (start 150.114 81.28) (end 150.114 87.884) (width 0.8) (layer F.Cu) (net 13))
 (segment (start 150.114 87.884) (end 158.79 96.56) (width 0.8) (layer F.Cu) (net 13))
 (segment (start 131.826 77.83937) (end 133.99663 80.01) (width 0.8) (layer F.Cu) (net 14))
 (segment (start 131.826 76.708) (end 131.826 77.83937) (width 0.8) (layer F.Cu) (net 14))
 (segment (start 133.99663 80.01) (end 147.066 80.01) (width 0.8) (layer F.Cu) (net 14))
 (segment (start 147.066 80.01) (end 148.844 81.788) (width 0.8) (layer F.Cu) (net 14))
 (segment (start 148.844 81.788) (end 148.844 88.646) (width 0.8) (layer F.Cu) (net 14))
 (segment (start 148.844 88.646) (end 150.876 90.678) (width 0.8) (layer F.Cu) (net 14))
 (segment (start 150.876 90.678) (end 150.876 95.758) (width 0.8) (layer F.Cu) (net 14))
 (segment (start 150.876 95.758) (end 150.876 112.522) (width 0.8) (layer F.Cu) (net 14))
 (segment (start 158.79 120.436) (end 158.79 135.168) (width 0.8) (layer F.Cu) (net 14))
 (segment (start 150.876 112.522) (end 158.79 120.436) (width 0.8) (layer F.Cu) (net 14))
 (segment (start 158.79 79.542) (end 158.79 86.614) (width 0.8) (layer F.Cu) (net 15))
 (segment (start 145.288 66.04) (end 158.79 79.542) (width 0.8) (layer F.Cu) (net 15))
 (segment (start 132.588 66.04) (end 145.288 66.04) (width 0.8) (layer F.Cu) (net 15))
 (segment (start 131.826 69.088) (end 131.826 66.802) (width 0.8) (layer F.Cu) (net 15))
 (segment (start 131.826 66.802) (end 132.588 66.04) (width 0.8) (layer F.Cu) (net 15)))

